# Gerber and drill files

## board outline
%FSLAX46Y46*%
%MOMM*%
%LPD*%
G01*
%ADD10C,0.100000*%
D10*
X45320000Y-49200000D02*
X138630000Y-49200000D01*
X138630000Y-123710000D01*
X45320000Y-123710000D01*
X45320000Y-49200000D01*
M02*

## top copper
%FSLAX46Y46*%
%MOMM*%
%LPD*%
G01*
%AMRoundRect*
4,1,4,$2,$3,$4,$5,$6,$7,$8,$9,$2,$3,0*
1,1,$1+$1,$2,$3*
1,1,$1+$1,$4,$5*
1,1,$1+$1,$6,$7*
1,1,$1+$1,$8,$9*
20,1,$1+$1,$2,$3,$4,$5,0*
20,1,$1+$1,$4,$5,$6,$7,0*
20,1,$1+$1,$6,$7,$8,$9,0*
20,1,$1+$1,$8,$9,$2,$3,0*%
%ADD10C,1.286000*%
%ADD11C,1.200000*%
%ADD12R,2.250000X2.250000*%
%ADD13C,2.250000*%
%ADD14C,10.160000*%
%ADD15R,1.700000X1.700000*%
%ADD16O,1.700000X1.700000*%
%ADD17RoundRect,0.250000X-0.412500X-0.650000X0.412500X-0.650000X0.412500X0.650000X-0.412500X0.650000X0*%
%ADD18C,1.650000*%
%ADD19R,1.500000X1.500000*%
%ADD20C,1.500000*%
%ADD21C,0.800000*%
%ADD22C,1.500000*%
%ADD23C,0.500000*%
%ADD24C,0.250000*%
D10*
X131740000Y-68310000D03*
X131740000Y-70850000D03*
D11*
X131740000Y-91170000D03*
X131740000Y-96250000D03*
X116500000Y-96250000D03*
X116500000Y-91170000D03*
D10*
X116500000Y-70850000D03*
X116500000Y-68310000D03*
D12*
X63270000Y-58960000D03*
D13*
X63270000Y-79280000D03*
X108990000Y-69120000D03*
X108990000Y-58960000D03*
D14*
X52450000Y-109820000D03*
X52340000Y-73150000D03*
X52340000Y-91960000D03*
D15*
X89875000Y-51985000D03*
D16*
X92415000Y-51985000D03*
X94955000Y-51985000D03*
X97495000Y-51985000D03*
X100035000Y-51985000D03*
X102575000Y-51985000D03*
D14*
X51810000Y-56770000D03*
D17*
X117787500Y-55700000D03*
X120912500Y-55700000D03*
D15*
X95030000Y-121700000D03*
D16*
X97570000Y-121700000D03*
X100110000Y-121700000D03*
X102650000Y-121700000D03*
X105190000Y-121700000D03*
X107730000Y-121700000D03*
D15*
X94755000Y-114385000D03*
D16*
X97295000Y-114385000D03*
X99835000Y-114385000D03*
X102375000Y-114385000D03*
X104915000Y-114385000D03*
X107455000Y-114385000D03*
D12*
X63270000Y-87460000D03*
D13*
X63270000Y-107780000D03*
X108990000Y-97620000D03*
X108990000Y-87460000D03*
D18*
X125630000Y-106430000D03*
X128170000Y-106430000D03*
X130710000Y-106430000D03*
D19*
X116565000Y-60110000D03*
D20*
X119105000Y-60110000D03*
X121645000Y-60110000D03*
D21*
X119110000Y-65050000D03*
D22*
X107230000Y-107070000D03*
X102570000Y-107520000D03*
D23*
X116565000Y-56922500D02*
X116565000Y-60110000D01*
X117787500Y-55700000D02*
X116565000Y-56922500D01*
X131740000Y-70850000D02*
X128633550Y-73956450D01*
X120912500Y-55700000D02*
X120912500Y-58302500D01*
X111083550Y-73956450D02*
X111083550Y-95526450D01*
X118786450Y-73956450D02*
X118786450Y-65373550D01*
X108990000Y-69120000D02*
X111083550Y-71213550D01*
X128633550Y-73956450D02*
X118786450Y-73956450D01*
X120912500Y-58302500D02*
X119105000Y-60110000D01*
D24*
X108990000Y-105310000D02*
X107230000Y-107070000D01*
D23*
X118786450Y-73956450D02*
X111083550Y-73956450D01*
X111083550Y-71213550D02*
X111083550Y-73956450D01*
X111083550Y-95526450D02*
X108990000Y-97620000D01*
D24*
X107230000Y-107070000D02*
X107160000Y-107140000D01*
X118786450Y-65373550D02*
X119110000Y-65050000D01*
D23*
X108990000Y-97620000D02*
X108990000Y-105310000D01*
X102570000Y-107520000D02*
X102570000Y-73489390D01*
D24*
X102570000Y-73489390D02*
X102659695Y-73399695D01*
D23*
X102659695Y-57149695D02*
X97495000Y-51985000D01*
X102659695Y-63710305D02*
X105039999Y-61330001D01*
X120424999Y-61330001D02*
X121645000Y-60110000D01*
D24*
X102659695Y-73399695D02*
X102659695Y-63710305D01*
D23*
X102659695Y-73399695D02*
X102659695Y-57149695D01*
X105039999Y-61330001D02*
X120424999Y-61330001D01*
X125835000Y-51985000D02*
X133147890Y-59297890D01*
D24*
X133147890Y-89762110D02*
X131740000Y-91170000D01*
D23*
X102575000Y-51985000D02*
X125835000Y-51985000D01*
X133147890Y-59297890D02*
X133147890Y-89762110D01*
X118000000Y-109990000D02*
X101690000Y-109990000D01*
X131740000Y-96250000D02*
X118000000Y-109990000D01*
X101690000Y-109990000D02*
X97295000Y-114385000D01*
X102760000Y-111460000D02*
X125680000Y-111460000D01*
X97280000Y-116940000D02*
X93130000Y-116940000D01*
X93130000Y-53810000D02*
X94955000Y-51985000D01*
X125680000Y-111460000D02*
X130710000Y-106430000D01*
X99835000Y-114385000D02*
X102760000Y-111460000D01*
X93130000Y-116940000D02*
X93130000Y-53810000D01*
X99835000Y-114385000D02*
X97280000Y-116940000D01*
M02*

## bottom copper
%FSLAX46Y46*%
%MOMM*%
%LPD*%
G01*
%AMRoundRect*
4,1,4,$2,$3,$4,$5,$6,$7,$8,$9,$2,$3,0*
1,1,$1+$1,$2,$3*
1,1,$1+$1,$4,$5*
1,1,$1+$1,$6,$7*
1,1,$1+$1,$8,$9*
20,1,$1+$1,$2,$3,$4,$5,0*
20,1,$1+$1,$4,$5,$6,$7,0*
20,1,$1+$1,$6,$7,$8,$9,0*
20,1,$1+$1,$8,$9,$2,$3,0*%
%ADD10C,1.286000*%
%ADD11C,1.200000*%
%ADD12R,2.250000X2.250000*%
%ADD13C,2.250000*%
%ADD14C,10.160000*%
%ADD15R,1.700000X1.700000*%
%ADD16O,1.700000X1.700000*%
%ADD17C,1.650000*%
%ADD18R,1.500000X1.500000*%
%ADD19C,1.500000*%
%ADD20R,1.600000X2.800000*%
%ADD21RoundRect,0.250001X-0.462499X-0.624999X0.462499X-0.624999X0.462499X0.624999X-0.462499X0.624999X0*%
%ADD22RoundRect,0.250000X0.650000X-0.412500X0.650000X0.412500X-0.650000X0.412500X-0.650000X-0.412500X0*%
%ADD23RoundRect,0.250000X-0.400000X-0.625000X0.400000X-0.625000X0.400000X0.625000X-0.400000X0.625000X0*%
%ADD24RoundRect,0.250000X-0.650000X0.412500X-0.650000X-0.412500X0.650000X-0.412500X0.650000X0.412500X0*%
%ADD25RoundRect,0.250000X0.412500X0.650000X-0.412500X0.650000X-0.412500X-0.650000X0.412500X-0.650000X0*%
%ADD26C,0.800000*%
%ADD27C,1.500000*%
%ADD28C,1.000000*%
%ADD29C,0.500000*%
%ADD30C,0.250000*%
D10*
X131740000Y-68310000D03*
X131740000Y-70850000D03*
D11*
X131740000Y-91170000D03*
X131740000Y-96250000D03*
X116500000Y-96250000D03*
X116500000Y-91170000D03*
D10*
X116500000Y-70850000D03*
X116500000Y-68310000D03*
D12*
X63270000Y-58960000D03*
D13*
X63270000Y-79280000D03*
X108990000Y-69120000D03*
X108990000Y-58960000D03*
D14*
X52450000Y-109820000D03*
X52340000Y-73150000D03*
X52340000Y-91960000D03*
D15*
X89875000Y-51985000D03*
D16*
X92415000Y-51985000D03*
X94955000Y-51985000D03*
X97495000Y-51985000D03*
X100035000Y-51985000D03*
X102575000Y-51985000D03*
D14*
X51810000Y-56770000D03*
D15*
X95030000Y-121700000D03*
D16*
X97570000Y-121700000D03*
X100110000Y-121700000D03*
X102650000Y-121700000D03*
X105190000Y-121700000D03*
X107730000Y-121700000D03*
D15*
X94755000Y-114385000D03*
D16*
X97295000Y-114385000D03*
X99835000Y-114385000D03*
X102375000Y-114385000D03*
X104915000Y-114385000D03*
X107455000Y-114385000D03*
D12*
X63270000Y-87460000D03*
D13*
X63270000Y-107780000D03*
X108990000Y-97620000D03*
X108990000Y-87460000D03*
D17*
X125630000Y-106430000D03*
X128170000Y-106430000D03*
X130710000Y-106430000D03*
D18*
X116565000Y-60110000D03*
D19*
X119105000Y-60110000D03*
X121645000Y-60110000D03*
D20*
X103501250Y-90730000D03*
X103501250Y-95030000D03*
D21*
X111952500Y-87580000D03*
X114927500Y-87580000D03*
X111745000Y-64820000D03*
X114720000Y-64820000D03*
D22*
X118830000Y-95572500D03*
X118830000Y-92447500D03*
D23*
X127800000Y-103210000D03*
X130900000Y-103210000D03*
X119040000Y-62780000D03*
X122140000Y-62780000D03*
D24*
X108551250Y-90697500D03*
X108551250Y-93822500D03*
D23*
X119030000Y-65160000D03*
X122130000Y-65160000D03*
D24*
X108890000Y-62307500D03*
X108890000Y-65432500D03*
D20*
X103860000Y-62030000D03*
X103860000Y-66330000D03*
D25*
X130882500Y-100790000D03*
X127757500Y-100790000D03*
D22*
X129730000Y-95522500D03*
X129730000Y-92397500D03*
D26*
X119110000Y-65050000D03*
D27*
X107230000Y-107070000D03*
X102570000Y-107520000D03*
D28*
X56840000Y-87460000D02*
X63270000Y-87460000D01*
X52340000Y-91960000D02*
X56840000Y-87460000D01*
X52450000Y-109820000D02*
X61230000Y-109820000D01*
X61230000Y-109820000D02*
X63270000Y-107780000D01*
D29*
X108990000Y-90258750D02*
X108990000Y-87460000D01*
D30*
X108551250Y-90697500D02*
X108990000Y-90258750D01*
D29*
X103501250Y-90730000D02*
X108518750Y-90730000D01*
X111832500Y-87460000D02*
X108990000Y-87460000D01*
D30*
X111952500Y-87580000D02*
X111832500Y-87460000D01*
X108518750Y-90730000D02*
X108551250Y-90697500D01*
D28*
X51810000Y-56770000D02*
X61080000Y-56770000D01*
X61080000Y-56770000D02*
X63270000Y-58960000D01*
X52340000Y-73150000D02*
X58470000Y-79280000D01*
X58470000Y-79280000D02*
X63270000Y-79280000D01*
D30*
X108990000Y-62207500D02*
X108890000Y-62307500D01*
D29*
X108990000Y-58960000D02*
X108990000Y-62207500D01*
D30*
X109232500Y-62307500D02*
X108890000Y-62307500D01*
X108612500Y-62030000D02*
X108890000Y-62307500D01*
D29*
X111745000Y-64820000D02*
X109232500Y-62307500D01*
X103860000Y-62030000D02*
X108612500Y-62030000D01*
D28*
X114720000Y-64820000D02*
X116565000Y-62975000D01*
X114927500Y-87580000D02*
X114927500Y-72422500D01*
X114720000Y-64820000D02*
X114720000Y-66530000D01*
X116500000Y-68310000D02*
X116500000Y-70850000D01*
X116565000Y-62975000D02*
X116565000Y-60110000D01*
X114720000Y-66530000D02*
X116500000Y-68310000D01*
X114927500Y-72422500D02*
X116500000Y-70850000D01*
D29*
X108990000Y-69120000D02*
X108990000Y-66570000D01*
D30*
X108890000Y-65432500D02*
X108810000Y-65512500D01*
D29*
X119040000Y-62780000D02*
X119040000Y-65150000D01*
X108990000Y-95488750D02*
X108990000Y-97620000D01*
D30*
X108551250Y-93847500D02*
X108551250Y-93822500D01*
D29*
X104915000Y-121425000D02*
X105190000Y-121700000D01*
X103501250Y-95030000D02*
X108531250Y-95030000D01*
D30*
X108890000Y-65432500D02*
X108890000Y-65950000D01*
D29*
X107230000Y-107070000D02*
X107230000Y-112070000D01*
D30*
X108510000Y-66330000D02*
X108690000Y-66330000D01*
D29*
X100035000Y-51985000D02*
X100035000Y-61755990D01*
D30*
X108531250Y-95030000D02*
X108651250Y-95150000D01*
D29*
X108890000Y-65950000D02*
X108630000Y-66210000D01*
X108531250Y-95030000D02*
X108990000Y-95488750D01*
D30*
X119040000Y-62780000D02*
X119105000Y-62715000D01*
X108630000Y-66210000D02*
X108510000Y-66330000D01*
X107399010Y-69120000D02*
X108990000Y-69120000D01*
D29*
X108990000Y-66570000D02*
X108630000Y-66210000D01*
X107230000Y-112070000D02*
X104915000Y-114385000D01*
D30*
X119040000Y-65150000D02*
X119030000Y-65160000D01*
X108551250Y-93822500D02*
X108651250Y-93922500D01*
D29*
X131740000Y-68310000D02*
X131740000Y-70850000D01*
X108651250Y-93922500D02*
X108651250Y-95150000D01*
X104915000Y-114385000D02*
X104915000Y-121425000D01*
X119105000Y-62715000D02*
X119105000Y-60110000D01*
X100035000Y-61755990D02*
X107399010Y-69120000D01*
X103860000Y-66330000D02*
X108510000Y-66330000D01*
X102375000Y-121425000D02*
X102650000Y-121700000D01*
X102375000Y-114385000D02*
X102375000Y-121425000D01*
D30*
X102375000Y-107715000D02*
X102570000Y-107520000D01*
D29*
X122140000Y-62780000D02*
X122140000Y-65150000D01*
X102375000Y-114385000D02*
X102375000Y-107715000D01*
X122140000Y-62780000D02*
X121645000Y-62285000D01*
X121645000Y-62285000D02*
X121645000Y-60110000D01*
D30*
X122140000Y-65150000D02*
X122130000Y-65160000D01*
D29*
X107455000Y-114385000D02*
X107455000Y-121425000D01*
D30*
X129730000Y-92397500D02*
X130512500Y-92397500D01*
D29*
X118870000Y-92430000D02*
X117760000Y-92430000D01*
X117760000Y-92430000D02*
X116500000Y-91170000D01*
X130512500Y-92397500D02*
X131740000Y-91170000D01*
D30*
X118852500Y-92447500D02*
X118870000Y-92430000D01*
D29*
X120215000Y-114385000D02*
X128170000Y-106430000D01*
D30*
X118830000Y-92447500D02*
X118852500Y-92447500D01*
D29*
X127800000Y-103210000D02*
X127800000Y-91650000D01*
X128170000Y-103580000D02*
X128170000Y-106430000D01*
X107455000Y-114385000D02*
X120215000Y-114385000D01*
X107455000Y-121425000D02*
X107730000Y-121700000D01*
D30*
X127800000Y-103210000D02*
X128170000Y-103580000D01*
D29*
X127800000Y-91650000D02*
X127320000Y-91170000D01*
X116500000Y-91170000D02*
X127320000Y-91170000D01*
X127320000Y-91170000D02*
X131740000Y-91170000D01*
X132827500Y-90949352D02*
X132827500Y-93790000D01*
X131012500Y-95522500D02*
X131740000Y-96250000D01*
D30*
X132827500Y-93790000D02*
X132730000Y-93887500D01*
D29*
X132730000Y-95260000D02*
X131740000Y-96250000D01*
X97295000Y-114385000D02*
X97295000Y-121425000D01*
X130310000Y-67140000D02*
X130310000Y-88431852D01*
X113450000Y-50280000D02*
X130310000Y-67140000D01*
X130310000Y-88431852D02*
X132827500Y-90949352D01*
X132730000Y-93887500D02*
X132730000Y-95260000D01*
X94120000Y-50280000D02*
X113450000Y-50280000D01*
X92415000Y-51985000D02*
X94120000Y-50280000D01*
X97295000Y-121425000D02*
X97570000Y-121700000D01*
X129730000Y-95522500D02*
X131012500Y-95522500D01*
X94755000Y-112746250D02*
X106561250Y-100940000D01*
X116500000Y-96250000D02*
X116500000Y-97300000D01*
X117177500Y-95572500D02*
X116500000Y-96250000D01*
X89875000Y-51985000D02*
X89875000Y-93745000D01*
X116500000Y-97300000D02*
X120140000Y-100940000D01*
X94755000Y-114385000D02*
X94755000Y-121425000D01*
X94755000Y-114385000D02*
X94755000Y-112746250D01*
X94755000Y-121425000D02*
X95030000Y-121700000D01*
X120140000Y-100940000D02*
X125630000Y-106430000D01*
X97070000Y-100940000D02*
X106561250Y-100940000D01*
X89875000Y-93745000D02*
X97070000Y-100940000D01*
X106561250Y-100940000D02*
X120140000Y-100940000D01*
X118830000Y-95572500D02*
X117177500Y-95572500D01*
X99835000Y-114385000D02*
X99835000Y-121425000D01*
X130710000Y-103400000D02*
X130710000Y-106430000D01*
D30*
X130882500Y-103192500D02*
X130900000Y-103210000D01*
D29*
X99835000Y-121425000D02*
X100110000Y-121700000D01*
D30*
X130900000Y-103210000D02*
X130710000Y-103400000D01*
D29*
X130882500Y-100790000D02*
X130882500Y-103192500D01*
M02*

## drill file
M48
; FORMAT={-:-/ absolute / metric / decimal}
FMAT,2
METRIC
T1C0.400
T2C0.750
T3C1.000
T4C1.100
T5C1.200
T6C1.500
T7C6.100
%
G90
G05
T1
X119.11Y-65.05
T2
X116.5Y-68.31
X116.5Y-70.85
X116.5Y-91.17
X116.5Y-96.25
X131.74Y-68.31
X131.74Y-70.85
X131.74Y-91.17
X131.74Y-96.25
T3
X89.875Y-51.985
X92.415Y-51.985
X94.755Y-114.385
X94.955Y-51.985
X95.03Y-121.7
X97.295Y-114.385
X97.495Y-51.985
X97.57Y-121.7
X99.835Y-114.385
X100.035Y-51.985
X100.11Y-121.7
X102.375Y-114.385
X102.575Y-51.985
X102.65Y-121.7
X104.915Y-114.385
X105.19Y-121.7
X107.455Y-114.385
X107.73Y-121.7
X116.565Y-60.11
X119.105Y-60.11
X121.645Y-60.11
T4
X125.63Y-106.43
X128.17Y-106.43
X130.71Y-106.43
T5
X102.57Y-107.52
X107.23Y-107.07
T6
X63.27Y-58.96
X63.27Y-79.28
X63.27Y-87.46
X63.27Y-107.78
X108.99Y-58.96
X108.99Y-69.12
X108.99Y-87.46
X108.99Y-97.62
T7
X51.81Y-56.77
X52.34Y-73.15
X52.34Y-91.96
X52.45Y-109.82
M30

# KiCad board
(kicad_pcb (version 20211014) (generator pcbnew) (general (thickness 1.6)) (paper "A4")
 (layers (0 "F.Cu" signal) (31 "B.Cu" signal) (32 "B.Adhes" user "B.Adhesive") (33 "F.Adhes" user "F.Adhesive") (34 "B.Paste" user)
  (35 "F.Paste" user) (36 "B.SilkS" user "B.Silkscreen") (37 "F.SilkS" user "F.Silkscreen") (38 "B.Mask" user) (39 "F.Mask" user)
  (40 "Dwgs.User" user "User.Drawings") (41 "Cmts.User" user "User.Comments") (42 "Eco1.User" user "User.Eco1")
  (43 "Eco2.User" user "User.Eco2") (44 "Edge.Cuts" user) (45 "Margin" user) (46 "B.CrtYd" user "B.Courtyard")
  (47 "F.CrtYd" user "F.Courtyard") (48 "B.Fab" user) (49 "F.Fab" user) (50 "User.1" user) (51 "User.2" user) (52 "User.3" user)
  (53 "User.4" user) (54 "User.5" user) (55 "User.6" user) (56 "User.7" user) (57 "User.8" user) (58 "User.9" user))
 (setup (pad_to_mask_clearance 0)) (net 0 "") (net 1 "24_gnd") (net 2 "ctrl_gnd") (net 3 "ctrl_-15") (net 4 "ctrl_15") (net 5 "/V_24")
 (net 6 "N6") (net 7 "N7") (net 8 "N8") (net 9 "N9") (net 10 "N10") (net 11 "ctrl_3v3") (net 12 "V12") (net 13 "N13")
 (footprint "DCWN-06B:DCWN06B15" (layer "F.Cu") (at 124.12 82.28)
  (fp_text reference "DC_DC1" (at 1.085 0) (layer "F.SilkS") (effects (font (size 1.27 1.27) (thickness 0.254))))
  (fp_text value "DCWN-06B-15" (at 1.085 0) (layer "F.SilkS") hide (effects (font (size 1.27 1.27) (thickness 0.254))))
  (pad "2" thru_hole circle (at 7.62 -13.97) (size 1.286 1.286) (drill 0.75) (layers *.Cu *.Mask) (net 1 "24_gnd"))
  (pad "3" thru_hole circle (at 7.62 -11.43) (size 1.286 1.286) (drill 0.75) (layers *.Cu *.Mask) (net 1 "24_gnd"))
  (pad "9" thru_hole circle (at 7.62 8.89) (size 1.2 1.2) (drill 0.75) (layers *.Cu *.Mask) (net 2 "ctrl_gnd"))
  (pad "11" thru_hole circle (at 7.62 13.97) (size 1.2 1.2) (drill 0.75) (layers *.Cu *.Mask) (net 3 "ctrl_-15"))
  (pad "14" thru_hole circle (at -7.62 13.97) (size 1.2 1.2) (drill 0.75) (layers *.Cu *.Mask) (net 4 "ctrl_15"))
  (pad "16" thru_hole circle (at -7.62 8.89) (size 1.2 1.2) (drill 0.75) (layers *.Cu *.Mask) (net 2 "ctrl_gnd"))
  (pad "22" thru_hole circle (at -7.62 -11.43) (size 1.286 1.286) (drill 0.75) (layers *.Cu *.Mask) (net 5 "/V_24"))
  (pad "23" thru_hole circle (at -7.62 -13.97) (size 1.286 1.286) (drill 0.75) (layers *.Cu *.Mask) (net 5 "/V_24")))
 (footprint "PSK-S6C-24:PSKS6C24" (layer "F.Cu") (at 63.27 58.96)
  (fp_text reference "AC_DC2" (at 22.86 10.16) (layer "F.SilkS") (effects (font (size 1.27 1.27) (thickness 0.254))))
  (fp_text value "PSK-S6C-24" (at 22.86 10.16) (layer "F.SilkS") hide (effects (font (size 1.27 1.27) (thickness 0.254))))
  (pad "1" thru_hole rect (at 0 0) (size 2.25 2.25) (drill 1.5) (layers *.Cu *.Mask) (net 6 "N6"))
  (pad "2" thru_hole circle (at 0 20.32) (size 2.25 2.25) (drill 1.5) (layers *.Cu *.Mask) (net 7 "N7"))
  (pad "3" thru_hole circle (at 45.72 10.16) (size 2.25 2.25) (drill 1.5) (layers *.Cu *.Mask) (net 1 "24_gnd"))
  (pad "4" thru_hole circle (at 45.72 0) (size 2.25 2.25) (drill 1.5) (layers *.Cu *.Mask) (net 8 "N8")))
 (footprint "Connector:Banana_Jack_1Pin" (layer "F.Cu") (at 52.45 109.82)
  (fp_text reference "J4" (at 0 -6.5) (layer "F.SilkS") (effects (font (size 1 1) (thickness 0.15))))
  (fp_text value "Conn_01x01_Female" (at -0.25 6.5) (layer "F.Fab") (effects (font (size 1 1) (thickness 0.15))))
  (pad "1" thru_hole circle (at 0 0) (size 10.16 10.16) (drill 6.1) (layers *.Cu *.Mask) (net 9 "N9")))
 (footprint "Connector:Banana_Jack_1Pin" (layer "F.Cu") (at 52.34 73.15)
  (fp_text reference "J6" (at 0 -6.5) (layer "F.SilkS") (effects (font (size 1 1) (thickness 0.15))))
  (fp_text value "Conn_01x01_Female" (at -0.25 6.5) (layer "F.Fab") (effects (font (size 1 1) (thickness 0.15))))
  (pad "1" thru_hole circle (at 0 0) (size 10.16 10.16) (drill 6.1) (layers *.Cu *.Mask) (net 7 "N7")))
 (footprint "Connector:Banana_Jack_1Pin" (layer "F.Cu") (at 52.34 91.96)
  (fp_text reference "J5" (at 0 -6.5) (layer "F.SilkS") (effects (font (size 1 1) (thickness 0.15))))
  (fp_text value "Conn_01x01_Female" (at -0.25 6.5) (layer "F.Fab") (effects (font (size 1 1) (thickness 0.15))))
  (pad "1" thru_hole circle (at 0 0) (size 10.16 10.16) (drill 6.1) (layers *.Cu *.Mask) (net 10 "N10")))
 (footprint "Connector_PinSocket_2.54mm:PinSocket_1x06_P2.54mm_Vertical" (layer "F.Cu") (at 89.875 51.985 90)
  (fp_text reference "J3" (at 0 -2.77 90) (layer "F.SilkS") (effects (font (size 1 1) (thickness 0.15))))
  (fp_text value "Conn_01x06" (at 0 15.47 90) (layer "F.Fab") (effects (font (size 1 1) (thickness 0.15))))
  (pad "1" thru_hole rect (at 0 0 90) (size 1.7 1.7) (drill 1) (layers *.Cu *.Mask) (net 4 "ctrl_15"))
  (pad "2" thru_hole oval (at 0 2.54 90) (size 1.7 1.7) (drill 1) (layers *.Cu *.Mask) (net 3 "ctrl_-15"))
  (pad "3" thru_hole oval (at 0 5.08 90) (size 1.7 1.7) (drill 1) (layers *.Cu *.Mask) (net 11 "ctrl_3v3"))
  (pad "4" thru_hole oval (at 0 7.62 90) (size 1.7 1.7) (drill 1) (layers *.Cu *.Mask) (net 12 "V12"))
  (pad "5" thru_hole oval (at 0 10.16 90) (size 1.7 1.7) (drill 1) (layers *.Cu *.Mask) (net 1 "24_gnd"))
  (pad "6" thru_hole oval (at 0 12.7 90) (size 1.7 1.7) (drill 1) (layers *.Cu *.Mask) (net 2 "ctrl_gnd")))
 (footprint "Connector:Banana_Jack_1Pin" (layer "F.Cu") (at 51.81 56.77)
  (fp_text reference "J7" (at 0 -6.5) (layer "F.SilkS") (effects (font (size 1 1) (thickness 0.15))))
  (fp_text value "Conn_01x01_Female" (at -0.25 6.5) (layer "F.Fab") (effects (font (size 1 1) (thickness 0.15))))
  (pad "1" thru_hole circle (at 0 0) (size 10.16 10.16) (drill 6.1) (layers *.Cu *.Mask) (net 6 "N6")))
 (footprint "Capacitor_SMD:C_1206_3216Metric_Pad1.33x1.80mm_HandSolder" (layer "F.Cu") (at 119.35 55.7)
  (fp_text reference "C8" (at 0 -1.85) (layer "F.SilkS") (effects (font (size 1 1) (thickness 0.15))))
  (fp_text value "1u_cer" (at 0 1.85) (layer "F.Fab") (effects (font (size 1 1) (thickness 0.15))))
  (pad "1" smd roundrect (at -1.5625 0) (size 1.325 1.8) (layers "F.Cu" "F.Paste" "F.Mask") (roundrect_rratio 0.188679) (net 5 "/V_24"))
  (pad "2" smd roundrect (at 1.5625 0) (size 1.325 1.8) (layers "F.Cu" "F.Paste" "F.Mask") (roundrect_rratio 0.188679) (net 1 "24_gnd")))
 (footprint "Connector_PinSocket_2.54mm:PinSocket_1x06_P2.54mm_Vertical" (layer "F.Cu") (at 95.03 121.7 90)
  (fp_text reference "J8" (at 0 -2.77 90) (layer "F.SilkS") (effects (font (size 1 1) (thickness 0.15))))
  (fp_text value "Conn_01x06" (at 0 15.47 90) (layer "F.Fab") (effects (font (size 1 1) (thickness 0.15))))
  (pad "1" thru_hole rect (at 0 0 90) (size 1.7 1.7) (drill 1) (layers *.Cu *.Mask) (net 4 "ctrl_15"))
  (pad "2" thru_hole oval (at 0 2.54 90) (size 1.7 1.7) (drill 1) (layers *.Cu *.Mask) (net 3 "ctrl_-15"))
  (pad "3" thru_hole oval (at 0 5.08 90) (size 1.7 1.7) (drill 1) (layers *.Cu *.Mask) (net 11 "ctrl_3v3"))
  (pad "4" thru_hole oval (at 0 7.62 90) (size 1.7 1.7) (drill 1) (layers *.Cu *.Mask) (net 12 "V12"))
  (pad "5" thru_hole oval (at 0 10.16 90) (size 1.7 1.7) (drill 1) (layers *.Cu *.Mask) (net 1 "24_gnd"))
  (pad "6" thru_hole oval (at 0 12.7 90) (size 1.7 1.7) (drill 1) (layers *.Cu *.Mask) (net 2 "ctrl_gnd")))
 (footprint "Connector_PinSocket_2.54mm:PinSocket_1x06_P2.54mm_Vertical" (layer "F.Cu") (at 94.755 114.385 90)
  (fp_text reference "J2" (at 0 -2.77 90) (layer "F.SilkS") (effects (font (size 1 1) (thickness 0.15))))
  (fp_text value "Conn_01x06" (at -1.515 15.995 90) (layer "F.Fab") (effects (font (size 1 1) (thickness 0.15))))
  (pad "1" thru_hole rect (at 0 0 90) (size 1.7 1.7) (drill 1) (layers *.Cu *.Mask) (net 4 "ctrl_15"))
  (pad "2" thru_hole oval (at 0 2.54 90) (size 1.7 1.7) (drill 1) (layers *.Cu *.Mask) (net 3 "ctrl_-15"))
  (pad "3" thru_hole oval (at 0 5.08 90) (size 1.7 1.7) (drill 1) (layers *.Cu *.Mask) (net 11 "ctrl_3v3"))
  (pad "4" thru_hole oval (at 0 7.62 90) (size 1.7 1.7) (drill 1) (layers *.Cu *.Mask) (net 12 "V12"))
  (pad "5" thru_hole oval (at 0 10.16 90) (size 1.7 1.7) (drill 1) (layers *.Cu *.Mask) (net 1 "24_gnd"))
  (pad "6" thru_hole oval (at 0 12.7 90) (size 1.7 1.7) (drill 1) (layers *.Cu *.Mask) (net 2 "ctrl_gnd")))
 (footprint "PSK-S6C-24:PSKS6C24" (layer "F.Cu") (at 63.27 87.46)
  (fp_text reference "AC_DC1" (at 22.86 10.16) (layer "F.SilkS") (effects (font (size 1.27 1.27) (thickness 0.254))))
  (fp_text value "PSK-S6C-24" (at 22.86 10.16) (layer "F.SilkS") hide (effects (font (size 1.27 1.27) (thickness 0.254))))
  (pad "1" thru_hole rect (at 0 0) (size 2.25 2.25) (drill 1.5) (layers *.Cu *.Mask) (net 10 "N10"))
  (pad "2" thru_hole circle (at 0 20.32) (size 2.25 2.25) (drill 1.5) (layers *.Cu *.Mask) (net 9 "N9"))
  (pad "3" thru_hole circle (at 45.72 10.16) (size 2.25 2.25) (drill 1.5) (layers *.Cu *.Mask) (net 1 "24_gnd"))
  (pad "4" thru_hole circle (at 45.72 0) (size 2.25 2.25) (drill 1.5) (layers *.Cu *.Mask) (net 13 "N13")))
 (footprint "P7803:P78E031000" (layer "F.Cu") (at 125.63 106.43)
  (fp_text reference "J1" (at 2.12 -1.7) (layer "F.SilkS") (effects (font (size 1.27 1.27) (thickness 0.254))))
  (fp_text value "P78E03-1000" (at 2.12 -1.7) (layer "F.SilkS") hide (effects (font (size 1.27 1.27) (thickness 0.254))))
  (pad "1" thru_hole circle (at 0 0) (size 1.65 1.65) (drill 1.1) (layers *.Cu *.Mask) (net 4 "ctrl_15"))
  (pad "2" thru_hole circle (at 2.54 0) (size 1.65 1.65) (drill 1.1) (layers *.Cu *.Mask) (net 2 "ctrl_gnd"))
  (pad "3" thru_hole circle (at 5.08 0) (size 1.65 1.65) (drill 1.1) (layers *.Cu *.Mask) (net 11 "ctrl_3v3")))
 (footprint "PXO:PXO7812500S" (layer "F.Cu") (at 116.565 60.11)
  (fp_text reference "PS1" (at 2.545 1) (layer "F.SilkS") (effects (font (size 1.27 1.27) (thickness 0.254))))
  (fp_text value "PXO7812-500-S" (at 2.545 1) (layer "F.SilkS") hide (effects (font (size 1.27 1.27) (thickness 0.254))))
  (pad "1" thru_hole rect (at 0 0) (size 1.5 1.5) (drill 1) (layers *.Cu *.Mask) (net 5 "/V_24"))
  (pad "2" thru_hole circle (at 2.54 0) (size 1.5 1.5) (drill 1) (layers *.Cu *.Mask) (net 1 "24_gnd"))
  (pad "3" thru_hole circle (at 5.08 0) (size 1.5 1.5) (drill 1) (layers *.Cu *.Mask) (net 12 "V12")))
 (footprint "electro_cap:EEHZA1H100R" (layer "B.Cu") (at 103.50125 92.88 -90)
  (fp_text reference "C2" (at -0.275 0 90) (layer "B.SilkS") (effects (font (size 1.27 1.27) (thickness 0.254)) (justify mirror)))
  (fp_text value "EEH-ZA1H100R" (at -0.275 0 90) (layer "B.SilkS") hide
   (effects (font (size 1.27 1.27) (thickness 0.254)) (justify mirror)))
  (pad "1" smd rect (at -2.15 0 180) (size 1.6 2.8) (layers "B.Cu" "B.Paste" "B.Mask") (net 13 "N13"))
  (pad "2" smd rect (at 2.15 0 180) (size 1.6 2.8) (layers "B.Cu" "B.Paste" "B.Mask") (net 1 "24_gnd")))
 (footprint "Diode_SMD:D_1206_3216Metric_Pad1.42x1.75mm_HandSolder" (layer "B.Cu") (at 113.44 87.58)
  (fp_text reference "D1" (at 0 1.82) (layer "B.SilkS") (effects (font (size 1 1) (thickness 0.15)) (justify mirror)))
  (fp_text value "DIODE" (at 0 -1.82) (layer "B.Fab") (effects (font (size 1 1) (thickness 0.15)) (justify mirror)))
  (pad "1" smd roundrect (at -1.4875 0) (size 1.425 1.75) (layers "B.Cu" "B.Paste" "B.Mask") (roundrect_rratio 0.175439) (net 13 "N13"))
  (pad "2" smd roundrect (at 1.4875 0) (size 1.425 1.75) (layers "B.Cu" "B.Paste" "B.Mask") (roundrect_rratio 0.175439) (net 5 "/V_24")))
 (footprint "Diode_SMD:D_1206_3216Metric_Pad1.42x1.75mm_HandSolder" (layer "B.Cu") (at 113.2325 64.82)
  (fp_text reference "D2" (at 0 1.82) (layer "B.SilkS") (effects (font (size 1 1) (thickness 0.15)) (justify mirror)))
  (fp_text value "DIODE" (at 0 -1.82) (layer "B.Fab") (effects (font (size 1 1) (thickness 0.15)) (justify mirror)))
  (pad "1" smd roundrect (at -1.4875 0) (size 1.425 1.75) (layers "B.Cu" "B.Paste" "B.Mask") (roundrect_rratio 0.175439) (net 8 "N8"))
  (pad "2" smd roundrect (at 1.4875 0) (size 1.425 1.75) (layers "B.Cu" "B.Paste" "B.Mask") (roundrect_rratio 0.175439) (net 5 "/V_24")))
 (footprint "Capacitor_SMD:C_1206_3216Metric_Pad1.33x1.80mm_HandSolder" (layer "B.Cu") (at 118.83 94.01 90)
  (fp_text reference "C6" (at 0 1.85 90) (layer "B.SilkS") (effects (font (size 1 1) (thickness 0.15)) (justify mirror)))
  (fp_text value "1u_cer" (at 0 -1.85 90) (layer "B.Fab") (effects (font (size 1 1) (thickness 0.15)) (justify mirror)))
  (pad "1" smd roundrect (at -1.5625 0 90) (size 1.325 1.8) (layers "B.Cu" "B.Paste" "B.Mask") (roundrect_rratio 0.188679) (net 4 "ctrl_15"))
  (pad "2" smd roundrect (at 1.5625 0 90) (size 1.325 1.8) (layers "B.Cu" "B.Paste" "B.Mask") (roundrect_rratio 0.188679) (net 2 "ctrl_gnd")))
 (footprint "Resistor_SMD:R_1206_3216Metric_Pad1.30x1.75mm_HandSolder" (layer "B.Cu") (at 129.35 103.21)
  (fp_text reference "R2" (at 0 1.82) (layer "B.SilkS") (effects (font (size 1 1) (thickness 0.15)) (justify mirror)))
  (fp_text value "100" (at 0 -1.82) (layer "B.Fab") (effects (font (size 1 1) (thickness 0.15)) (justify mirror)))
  (pad "1" smd roundrect (at -1.55 0) (size 1.3 1.75) (layers "B.Cu" "B.Paste" "B.Mask") (roundrect_rratio 0.192308) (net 2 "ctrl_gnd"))
  (pad "2" smd roundrect (at 1.55 0) (size 1.3 1.75) (layers "B.Cu" "B.Paste" "B.Mask") (roundrect_rratio 0.192308) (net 11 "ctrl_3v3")))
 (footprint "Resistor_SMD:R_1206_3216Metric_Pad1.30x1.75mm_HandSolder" (layer "B.Cu") (at 120.59 62.78)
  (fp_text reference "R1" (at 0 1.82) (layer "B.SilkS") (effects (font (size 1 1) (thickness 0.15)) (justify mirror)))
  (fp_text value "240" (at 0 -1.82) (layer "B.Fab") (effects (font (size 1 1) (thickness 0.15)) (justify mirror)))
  (pad "1" smd roundrect (at -1.55 0) (size 1.3 1.75) (layers "B.Cu" "B.Paste" "B.Mask") (roundrect_rratio 0.192308) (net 1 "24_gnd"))
  (pad "2" smd roundrect (at 1.55 0) (size 1.3 1.75) (layers "B.Cu" "B.Paste" "B.Mask") (roundrect_rratio 0.192308) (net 12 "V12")))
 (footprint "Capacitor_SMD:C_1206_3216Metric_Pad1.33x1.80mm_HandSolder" (layer "B.Cu") (at 108.55125 92.26 -90)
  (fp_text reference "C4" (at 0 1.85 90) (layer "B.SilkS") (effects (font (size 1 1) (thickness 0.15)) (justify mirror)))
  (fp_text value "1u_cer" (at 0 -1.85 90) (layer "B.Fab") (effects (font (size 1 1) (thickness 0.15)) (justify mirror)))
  (pad "1" smd roundrect (at -1.5625 0 270) (size 1.325 1.8) (layers "B.Cu" "B.Paste" "B.Mask") (roundrect_rratio 0.188679) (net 13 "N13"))
  (pad "2" smd roundrect (at 1.5625 0 270) (size 1.325 1.8) (layers "B.Cu" "B.Paste" "B.Mask") (roundrect_rratio 0.188679) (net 1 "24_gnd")))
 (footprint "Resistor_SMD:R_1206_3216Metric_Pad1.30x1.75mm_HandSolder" (layer "B.Cu") (at 120.58 65.16)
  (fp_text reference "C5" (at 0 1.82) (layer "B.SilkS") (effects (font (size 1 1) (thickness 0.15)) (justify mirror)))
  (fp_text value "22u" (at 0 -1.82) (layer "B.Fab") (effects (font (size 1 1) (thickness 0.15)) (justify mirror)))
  (pad "1" smd roundrect (at -1.55 0) (size 1.3 1.75) (layers "B.Cu" "B.Paste" "B.Mask") (roundrect_rratio 0.192308) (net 1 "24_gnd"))
  (pad "2" smd roundrect (at 1.55 0) (size 1.3 1.75) (layers "B.Cu" "B.Paste" "B.Mask") (roundrect_rratio 0.192308) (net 12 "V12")))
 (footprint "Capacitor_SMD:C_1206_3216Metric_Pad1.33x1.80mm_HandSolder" (layer "B.Cu") (at 108.89 63.87 -90)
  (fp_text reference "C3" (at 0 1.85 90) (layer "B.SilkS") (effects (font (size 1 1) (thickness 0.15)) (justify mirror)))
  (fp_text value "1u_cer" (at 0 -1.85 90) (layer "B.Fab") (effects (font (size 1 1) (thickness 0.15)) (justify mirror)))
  (pad "1" smd roundrect (at -1.5625 0 270) (size 1.325 1.8) (layers "B.Cu" "B.Paste" "B.Mask") (roundrect_rratio 0.188679) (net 8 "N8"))
  (pad "2" smd roundrect (at 1.5625 0 270) (size 1.325 1.8) (layers "B.Cu" "B.Paste" "B.Mask") (roundrect_rratio 0.188679) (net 1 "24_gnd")))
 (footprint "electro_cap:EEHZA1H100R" (layer "B.Cu") (at 103.86 64.18 -90)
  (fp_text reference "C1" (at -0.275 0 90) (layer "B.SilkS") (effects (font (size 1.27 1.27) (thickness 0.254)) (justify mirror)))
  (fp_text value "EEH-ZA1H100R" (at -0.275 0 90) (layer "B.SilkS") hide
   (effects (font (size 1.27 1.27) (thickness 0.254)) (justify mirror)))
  (pad "1" smd rect (at -2.15 0 180) (size 1.6 2.8) (layers "B.Cu" "B.Paste" "B.Mask") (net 8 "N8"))
  (pad "2" smd rect (at 2.15 0 180) (size 1.6 2.8) (layers "B.Cu" "B.Paste" "B.Mask") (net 1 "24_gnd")))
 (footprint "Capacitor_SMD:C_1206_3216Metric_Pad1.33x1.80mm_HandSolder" (layer "B.Cu") (at 129.32 100.79 180)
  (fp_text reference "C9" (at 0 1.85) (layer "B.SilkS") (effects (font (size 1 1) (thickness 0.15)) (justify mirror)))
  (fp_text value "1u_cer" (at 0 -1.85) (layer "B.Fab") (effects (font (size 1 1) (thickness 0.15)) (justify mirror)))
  (pad "1" smd roundrect (at -1.5625 0 180) (size 1.325 1.8) (layers "B.Cu" "B.Paste" "B.Mask") (roundrect_rratio 0.188679)
   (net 11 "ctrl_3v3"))
  (pad "2" smd roundrect (at 1.5625 0 180) (size 1.325 1.8) (layers "B.Cu" "B.Paste" "B.Mask") (roundrect_rratio 0.188679)
   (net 2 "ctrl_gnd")))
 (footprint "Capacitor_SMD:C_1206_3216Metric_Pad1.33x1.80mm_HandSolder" (layer "B.Cu") (at 129.73 93.96 90)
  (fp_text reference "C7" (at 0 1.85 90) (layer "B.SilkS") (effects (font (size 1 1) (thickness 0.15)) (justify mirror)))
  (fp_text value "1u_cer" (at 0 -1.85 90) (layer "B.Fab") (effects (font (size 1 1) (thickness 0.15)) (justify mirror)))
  (pad "1" smd roundrect (at -1.5625 0 90) (size 1.325 1.8) (layers "B.Cu" "B.Paste" "B.Mask") (roundrect_rratio 0.188679)
   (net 3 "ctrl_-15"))
  (pad "2" smd roundrect (at 1.5625 0 90) (size 1.325 1.8) (layers "B.Cu" "B.Paste" "B.Mask") (roundrect_rratio 0.188679) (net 2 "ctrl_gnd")))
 (gr_rect (start 45.32 49.2) (end 138.63 123.71) (layer "Edge.Cuts") (width 0.1) (fill none))
 (segment (start 56.84 87.46) (end 63.27 87.46) (width 1) (layer "B.Cu") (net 10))
 (segment (start 52.34 91.96) (end 56.84 87.46) (width 1) (layer "B.Cu") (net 10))
 (segment (start 52.45 109.82) (end 61.23 109.82) (width 1) (layer "B.Cu") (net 9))
 (segment (start 61.23 109.82) (end 63.27 107.78) (width 1) (layer "B.Cu") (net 9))
 (segment (start 108.99 90.25875) (end 108.99 87.46) (width 0.5) (layer "B.Cu") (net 13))
 (segment (start 108.55125 90.6975) (end 108.99 90.25875) (width 0.25) (layer "B.Cu") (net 13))
 (segment (start 103.50125 90.73) (end 108.51875 90.73) (width 0.5) (layer "B.Cu") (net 13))
 (segment (start 111.8325 87.46) (end 108.99 87.46) (width 0.5) (layer "B.Cu") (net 13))
 (segment (start 111.9525 87.58) (end 111.8325 87.46) (width 0.25) (layer "B.Cu") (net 13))
 (segment (start 108.51875 90.73) (end 108.55125 90.6975) (width 0.25) (layer "B.Cu") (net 13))
 (segment (start 51.81 56.77) (end 61.08 56.77) (width 1) (layer "B.Cu") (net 6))
 (segment (start 61.08 56.77) (end 63.27 58.96) (width 1) (layer "B.Cu") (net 6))
 (segment (start 52.34 73.15) (end 58.47 79.28) (width 1) (layer "B.Cu") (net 7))
 (segment (start 58.47 79.28) (end 63.27 79.28) (width 1) (layer "B.Cu") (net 7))
 (segment (start 108.99 62.2075) (end 108.89 62.3075) (width 0.25) (layer "B.Cu") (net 8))
 (segment (start 108.99 58.96) (end 108.99 62.2075) (width 0.5) (layer "B.Cu") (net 8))
 (segment (start 109.2325 62.3075) (end 108.89 62.3075) (width 0.25) (layer "B.Cu") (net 8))
 (segment (start 108.6125 62.03) (end 108.89 62.3075) (width 0.25) (layer "B.Cu") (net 8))
 (segment (start 111.745 64.82) (end 109.2325 62.3075) (width 0.5) (layer "B.Cu") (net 8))
 (segment (start 103.86 62.03) (end 108.6125 62.03) (width 0.5) (layer "B.Cu") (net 8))
 (segment (start 116.565 56.9225) (end 116.565 60.11) (width 0.5) (layer "F.Cu") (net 5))
 (segment (start 117.7875 55.7) (end 116.565 56.9225) (width 0.5) (layer "F.Cu") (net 5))
 (segment (start 114.72 64.82) (end 116.565 62.975) (width 1) (layer "B.Cu") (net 5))
 (segment (start 114.9275 87.58) (end 114.9275 72.4225) (width 1) (layer "B.Cu") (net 5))
 (segment (start 114.72 64.82) (end 114.72 66.53) (width 1) (layer "B.Cu") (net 5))
 (segment (start 116.5 68.31) (end 116.5 70.85) (width 1) (layer "B.Cu") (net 5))
 (segment (start 116.565 62.975) (end 116.565 60.11) (width 1) (layer "B.Cu") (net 5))
 (segment (start 114.72 66.53) (end 116.5 68.31) (width 1) (layer "B.Cu") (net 5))
 (segment (start 114.9275 72.4225) (end 116.5 70.85) (width 1) (layer "B.Cu") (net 5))
 (segment (start 131.74 70.85) (end 128.63355 73.95645) (width 0.5) (layer "F.Cu") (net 1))
 (segment (start 120.9125 55.7) (end 120.9125 58.3025) (width 0.5) (layer "F.Cu") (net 1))
 (segment (start 111.08355 73.95645) (end 111.08355 95.52645) (width 0.5) (layer "F.Cu") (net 1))
 (segment (start 118.78645 73.95645) (end 118.78645 65.37355) (width 0.5) (layer "F.Cu") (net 1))
 (segment (start 108.99 69.12) (end 111.08355 71.21355) (width 0.5) (layer "F.Cu") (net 1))
 (segment (start 128.63355 73.95645) (end 118.78645 73.95645) (width 0.5) (layer "F.Cu") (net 1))
 (segment (start 120.9125 58.3025) (end 119.105 60.11) (width 0.5) (layer "F.Cu") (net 1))
 (segment (start 108.99 105.31) (end 107.23 107.07) (width 0.25) (layer "F.Cu") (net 1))
 (segment (start 118.78645 73.95645) (end 111.08355 73.95645) (width 0.5) (layer "F.Cu") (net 1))
 (segment (start 111.08355 71.21355) (end 111.08355 73.95645) (width 0.5) (layer "F.Cu") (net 1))
 (segment (start 111.08355 95.52645) (end 108.99 97.62) (width 0.5) (layer "F.Cu") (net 1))
 (segment (start 107.23 107.07) (end 107.16 107.14) (width 0.25) (layer "F.Cu") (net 1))
 (segment (start 118.78645 65.37355) (end 119.11 65.05) (width 0.25) (layer "F.Cu") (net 1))
 (segment (start 108.99 97.62) (end 108.99 105.31) (width 0.5) (layer "F.Cu") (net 1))
 (via (at 119.11 65.05) (size 0.8) (drill 0.4) (layers "F.Cu" "B.Cu") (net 1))
 (via (at 107.23 107.07) (size 1.5) (drill 1.2) (layers "F.Cu" "B.Cu") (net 1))
 (segment (start 108.99 69.12) (end 108.99 66.57) (width 0.5) (layer "B.Cu") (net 1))
 (segment (start 108.89 65.4325) (end 108.81 65.5125) (width 0.25) (layer "B.Cu") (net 1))
 (segment (start 119.04 62.78) (end 119.04 65.15) (width 0.5) (layer "B.Cu") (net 1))
 (segment (start 108.99 95.48875) (end 108.99 97.62) (width 0.5) (layer "B.Cu") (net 1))
 (segment (start 108.55125 93.8475) (end 108.55125 93.8225) (width 0.25) (layer "B.Cu") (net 1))
 (segment (start 104.915 121.425) (end 105.19 121.7) (width 0.5) (layer "B.Cu") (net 1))
 (segment (start 103.50125 95.03) (end 108.53125 95.03) (width 0.5) (layer "B.Cu") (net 1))
 (segment (start 108.89 65.4325) (end 108.89 65.95) (width 0.25) (layer "B.Cu") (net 1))
 (segment (start 107.23 107.07) (end 107.23 112.07) (width 0.5) (layer "B.Cu") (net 1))
 (segment (start 108.51 66.33) (end 108.69 66.33) (width 0.25) (layer "B.Cu") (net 1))
 (segment (start 100.035 51.985) (end 100.035 61.75599) (width 0.5) (layer "B.Cu") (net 1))
 (segment (start 108.53125 95.03) (end 108.65125 95.15) (width 0.25) (layer "B.Cu") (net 1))
 (segment (start 108.89 65.95) (end 108.63 66.21) (width 0.5) (layer "B.Cu") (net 1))
 (segment (start 108.53125 95.03) (end 108.99 95.48875) (width 0.5) (layer "B.Cu") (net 1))
 (segment (start 119.04 62.78) (end 119.105 62.715) (width 0.25) (layer "B.Cu") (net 1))
 (segment (start 108.63 66.21) (end 108.51 66.33) (width 0.25) (layer "B.Cu") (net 1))
 (segment (start 107.39901 69.12) (end 108.99 69.12) (width 0.25) (layer "B.Cu") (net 1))
 (segment (start 108.99 66.57) (end 108.63 66.21) (width 0.5) (layer "B.Cu") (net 1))
 (segment (start 107.23 112.07) (end 104.915 114.385) (width 0.5) (layer "B.Cu") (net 1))
 (segment (start 119.04 65.15) (end 119.03 65.16) (width 0.25) (layer "B.Cu") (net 1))
 (segment (start 108.55125 93.8225) (end 108.65125 93.9225) (width 0.25) (layer "B.Cu") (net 1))
 (segment (start 131.74 68.31) (end 131.74 70.85) (width 0.5) (layer "B.Cu") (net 1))
 (segment (start 108.65125 93.9225) (end 108.65125 95.15) (width 0.5) (layer "B.Cu") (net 1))
 (segment (start 104.915 114.385) (end 104.915 121.425) (width 0.5) (layer "B.Cu") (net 1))
 (segment (start 119.105 62.715) (end 119.105 60.11) (width 0.5) (layer "B.Cu") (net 1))
 (segment (start 100.035 61.75599) (end 107.39901 69.12) (width 0.5) (layer "B.Cu") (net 1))
 (segment (start 103.86 66.33) (end 108.51 66.33) (width 0.5) (layer "B.Cu") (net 1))
 (segment (start 102.57 107.52) (end 102.57 73.48939) (width 0.5) (layer "F.Cu") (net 12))
 (segment (start 102.57 73.48939) (end 102.659695 73.399695) (width 0.25) (layer "F.Cu") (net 12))
 (segment (start 102.659695 57.149695) (end 97.495 51.985) (width 0.5) (layer "F.Cu") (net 12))
 (segment (start 102.659695 63.710305) (end 105.039999 61.330001) (width 0.5) (layer "F.Cu") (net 12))
 (segment (start 120.424999 61.330001) (end 121.645 60.11) (width 0.5) (layer "F.Cu") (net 12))
 (segment (start 102.659695 73.399695) (end 102.659695 63.710305) (width 0.25) (layer "F.Cu") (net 12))
 (segment (start 102.659695 73.399695) (end 102.659695 57.149695) (width 0.5) (layer "F.Cu") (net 12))
 (segment (start 105.039999 61.330001) (end 120.424999 61.330001) (width 0.5) (layer "F.Cu") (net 12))
 (via (at 102.57 107.52) (size 1.5) (drill 1.2) (layers "F.Cu" "B.Cu") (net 12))
 (segment (start 102.375 121.425) (end 102.65 121.7) (width 0.5) (layer "B.Cu") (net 12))
 (segment (start 102.375 114.385) (end 102.375 121.425) (width 0.5) (layer "B.Cu") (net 12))
 (segment (start 102.375 107.715) (end 102.57 107.52) (width 0.25) (layer "B.Cu") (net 12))
 (segment (start 122.14 62.78) (end 122.14 65.15) (width 0.5) (layer "B.Cu") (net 12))
 (segment (start 102.375 114.385) (end 102.375 107.715) (width 0.5) (layer "B.Cu") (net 12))
 (segment (start 122.14 62.78) (end 121.645 62.285) (width 0.5) (layer "B.Cu") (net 12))
 (segment (start 121.645 62.285) (end 121.645 60.11) (width 0.5) (layer "B.Cu") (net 12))
 (segment (start 122.14 65.15) (end 122.13 65.16) (width 0.25) (layer "B.Cu") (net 12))
 (segment (start 125.835 51.985) (end 133.14789 59.29789) (width 0.5) (layer "F.Cu") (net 2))
 (segment (start 133.14789 89.76211) (end 131.74 91.17) (width 0.25) (layer "F.Cu") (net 2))
 (segment (start 102.575 51.985) (end 125.835 51.985) (width 0.5) (layer "F.Cu") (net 2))
 (segment (start 133.14789 59.29789) (end 133.14789 89.76211) (width 0.5) (layer "F.Cu") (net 2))
 (segment (start 107.455 114.385) (end 107.455 121.425) (width 0.5) (layer "B.Cu") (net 2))
 (segment (start 129.73 92.3975) (end 130.5125 92.3975) (width 0.25) (layer "B.Cu") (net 2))
 (segment (start 118.87 92.43) (end 117.76 92.43) (width 0.5) (layer "B.Cu") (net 2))
 (segment (start 117.76 92.43) (end 116.5 91.17) (width 0.5) (layer "B.Cu") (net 2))
 (segment (start 130.5125 92.3975) (end 131.74 91.17) (width 0.5) (layer "B.Cu") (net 2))
 (segment (start 118.8525 92.4475) (end 118.87 92.43) (width 0.25) (layer "B.Cu") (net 2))
 (segment (start 120.215 114.385) (end 128.17 106.43) (width 0.5) (layer "B.Cu") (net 2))
 (segment (start 118.83 92.4475) (end 118.8525 92.4475) (width 0.25) (layer "B.Cu") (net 2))
 (segment (start 127.8 103.21) (end 127.8 91.65) (width 0.5) (layer "B.Cu") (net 2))
 (segment (start 128.17 103.58) (end 128.17 106.43) (width 0.5) (layer "B.Cu") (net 2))
 (segment (start 107.455 114.385) (end 120.215 114.385) (width 0.5) (layer "B.Cu") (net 2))
 (segment (start 107.455 121.425) (end 107.73 121.7) (width 0.5) (layer "B.Cu") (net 2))
 (segment (start 127.8 103.21) (end 128.17 103.58) (width 0.25) (layer "B.Cu") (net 2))
 (segment (start 127.8 91.65) (end 127.32 91.17) (width 0.5) (layer "B.Cu") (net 2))
 (segment (start 116.5 91.17) (end 127.32 91.17) (width 0.5) (layer "B.Cu") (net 2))
 (segment (start 127.32 91.17) (end 131.74 91.17) (width 0.5) (layer "B.Cu") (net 2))
 (segment (start 118 109.99) (end 101.69 109.99) (width 0.5) (layer "F.Cu") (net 3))
 (segment (start 131.74 96.25) (end 118 109.99) (width 0.5) (layer "F.Cu") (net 3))
 (segment (start 101.69 109.99) (end 97.295 114.385) (width 0.5) (layer "F.Cu") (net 3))
 (segment (start 132.8275 90.949352) (end 132.8275 93.79) (width 0.5) (layer "B.Cu") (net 3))
 (segment (start 131.0125 95.5225) (end 131.74 96.25) (width 0.5) (layer "B.Cu") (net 3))
 (segment (start 132.8275 93.79) (end 132.73 93.8875) (width 0.25) (layer "B.Cu") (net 3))
 (segment (start 132.73 95.26) (end 131.74 96.25) (width 0.5) (layer "B.Cu") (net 3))
 (segment (start 97.295 114.385) (end 97.295 121.425) (width 0.5) (layer "B.Cu") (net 3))
 (segment (start 130.31 67.14) (end 130.31 88.431852) (width 0.5) (layer "B.Cu") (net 3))
 (segment (start 113.45 50.28) (end 130.31 67.14) (width 0.5) (layer "B.Cu") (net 3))
 (segment (start 130.31 88.431852) (end 132.8275 90.949352) (width 0.5) (layer "B.Cu") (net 3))
 (segment (start 132.73 93.8875) (end 132.73 95.26) (width 0.5) (layer "B.Cu") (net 3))
 (segment (start 94.12 50.28) (end 113.45 50.28) (width 0.5) (layer "B.Cu") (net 3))
 (segment (start 92.415 51.985) (end 94.12 50.28) (width 0.5) (layer "B.Cu") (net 3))
 (segment (start 97.295 121.425) (end 97.57 121.7) (width 0.5) (layer "B.Cu") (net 3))
 (segment (start 129.73 95.5225) (end 131.0125 95.5225) (width 0.5) (layer "B.Cu") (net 3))
 (segment (start 94.755 112.74625) (end 106.56125 100.94) (width 0.5) (layer "B.Cu") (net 4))
 (segment (start 116.5 96.25) (end 116.5 97.3) (width 0.5) (layer "B.Cu") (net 4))
 (segment (start 117.1775 95.5725) (end 116.5 96.25) (width 0.5) (layer "B.Cu") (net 4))
 (segment (start 89.875 51.985) (end 89.875 93.745) (width 0.5) (layer "B.Cu") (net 4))
 (segment (start 116.5 97.3) (end 120.14 100.94) (width 0.5) (layer "B.Cu") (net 4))
 (segment (start 94.755 114.385) (end 94.755 121.425) (width 0.5) (layer "B.Cu") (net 4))
 (segment (start 94.755 114.385) (end 94.755 112.74625) (width 0.5) (layer "B.Cu") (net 4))
 (segment (start 94.755 121.425) (end 95.03 121.7) (width 0.5) (layer "B.Cu") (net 4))
 (segment (start 120.14 100.94) (end 125.63 106.43) (width 0.5) (layer "B.Cu") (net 4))
 (segment (start 97.07 100.94) (end 106.56125 100.94) (width 0.5) (layer "B.Cu") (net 4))
 (segment (start 89.875 93.745) (end 97.07 100.94) (width 0.5) (layer "B.Cu") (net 4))
 (segment (start 106.56125 100.94) (end 120.14 100.94) (width 0.5) (layer "B.Cu") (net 4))
 (segment (start 118.83 95.5725) (end 117.1775 95.5725) (width 0.5) (layer "B.Cu") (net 4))
 (segment (start 102.76 111.46) (end 125.68 111.46) (width 0.5) (layer "F.Cu") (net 11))
 (segment (start 97.28 116.94) (end 93.13 116.94) (width 0.5) (layer "F.Cu") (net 11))
 (segment (start 93.13 53.81) (end 94.955 51.985) (width 0.5) (layer "F.Cu") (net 11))
 (segment (start 125.68 111.46) (end 130.71 106.43) (width 0.5) (layer "F.Cu") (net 11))
 (segment (start 99.835 114.385) (end 102.76 111.46) (width 0.5) (layer "F.Cu") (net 11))
 (segment (start 93.13 116.94) (end 93.13 53.81) (width 0.5) (layer "F.Cu") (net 11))
 (segment (start 99.835 114.385) (end 97.28 116.94) (width 0.5) (layer "F.Cu") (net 11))
 (segment (start 99.835 114.385) (end 99.835 121.425) (width 0.5) (layer "B.Cu") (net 11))
 (segment (start 130.71 103.4) (end 130.71 106.43) (width 0.5) (layer "B.Cu") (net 11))
 (segment (start 130.8825 103.1925) (end 130.9 103.21) (width 0.25) (layer "B.Cu") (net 11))
 (segment (start 99.835 121.425) (end 100.11 121.7) (width 0.5) (layer "B.Cu") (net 11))
 (segment (start 130.9 103.21) (end 130.71 103.4) (width 0.25) (layer "B.Cu") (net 11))
 (segment (start 130.8825 100.79) (end 130.8825 103.1925) (width 0.5) (layer "B.Cu") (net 11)))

